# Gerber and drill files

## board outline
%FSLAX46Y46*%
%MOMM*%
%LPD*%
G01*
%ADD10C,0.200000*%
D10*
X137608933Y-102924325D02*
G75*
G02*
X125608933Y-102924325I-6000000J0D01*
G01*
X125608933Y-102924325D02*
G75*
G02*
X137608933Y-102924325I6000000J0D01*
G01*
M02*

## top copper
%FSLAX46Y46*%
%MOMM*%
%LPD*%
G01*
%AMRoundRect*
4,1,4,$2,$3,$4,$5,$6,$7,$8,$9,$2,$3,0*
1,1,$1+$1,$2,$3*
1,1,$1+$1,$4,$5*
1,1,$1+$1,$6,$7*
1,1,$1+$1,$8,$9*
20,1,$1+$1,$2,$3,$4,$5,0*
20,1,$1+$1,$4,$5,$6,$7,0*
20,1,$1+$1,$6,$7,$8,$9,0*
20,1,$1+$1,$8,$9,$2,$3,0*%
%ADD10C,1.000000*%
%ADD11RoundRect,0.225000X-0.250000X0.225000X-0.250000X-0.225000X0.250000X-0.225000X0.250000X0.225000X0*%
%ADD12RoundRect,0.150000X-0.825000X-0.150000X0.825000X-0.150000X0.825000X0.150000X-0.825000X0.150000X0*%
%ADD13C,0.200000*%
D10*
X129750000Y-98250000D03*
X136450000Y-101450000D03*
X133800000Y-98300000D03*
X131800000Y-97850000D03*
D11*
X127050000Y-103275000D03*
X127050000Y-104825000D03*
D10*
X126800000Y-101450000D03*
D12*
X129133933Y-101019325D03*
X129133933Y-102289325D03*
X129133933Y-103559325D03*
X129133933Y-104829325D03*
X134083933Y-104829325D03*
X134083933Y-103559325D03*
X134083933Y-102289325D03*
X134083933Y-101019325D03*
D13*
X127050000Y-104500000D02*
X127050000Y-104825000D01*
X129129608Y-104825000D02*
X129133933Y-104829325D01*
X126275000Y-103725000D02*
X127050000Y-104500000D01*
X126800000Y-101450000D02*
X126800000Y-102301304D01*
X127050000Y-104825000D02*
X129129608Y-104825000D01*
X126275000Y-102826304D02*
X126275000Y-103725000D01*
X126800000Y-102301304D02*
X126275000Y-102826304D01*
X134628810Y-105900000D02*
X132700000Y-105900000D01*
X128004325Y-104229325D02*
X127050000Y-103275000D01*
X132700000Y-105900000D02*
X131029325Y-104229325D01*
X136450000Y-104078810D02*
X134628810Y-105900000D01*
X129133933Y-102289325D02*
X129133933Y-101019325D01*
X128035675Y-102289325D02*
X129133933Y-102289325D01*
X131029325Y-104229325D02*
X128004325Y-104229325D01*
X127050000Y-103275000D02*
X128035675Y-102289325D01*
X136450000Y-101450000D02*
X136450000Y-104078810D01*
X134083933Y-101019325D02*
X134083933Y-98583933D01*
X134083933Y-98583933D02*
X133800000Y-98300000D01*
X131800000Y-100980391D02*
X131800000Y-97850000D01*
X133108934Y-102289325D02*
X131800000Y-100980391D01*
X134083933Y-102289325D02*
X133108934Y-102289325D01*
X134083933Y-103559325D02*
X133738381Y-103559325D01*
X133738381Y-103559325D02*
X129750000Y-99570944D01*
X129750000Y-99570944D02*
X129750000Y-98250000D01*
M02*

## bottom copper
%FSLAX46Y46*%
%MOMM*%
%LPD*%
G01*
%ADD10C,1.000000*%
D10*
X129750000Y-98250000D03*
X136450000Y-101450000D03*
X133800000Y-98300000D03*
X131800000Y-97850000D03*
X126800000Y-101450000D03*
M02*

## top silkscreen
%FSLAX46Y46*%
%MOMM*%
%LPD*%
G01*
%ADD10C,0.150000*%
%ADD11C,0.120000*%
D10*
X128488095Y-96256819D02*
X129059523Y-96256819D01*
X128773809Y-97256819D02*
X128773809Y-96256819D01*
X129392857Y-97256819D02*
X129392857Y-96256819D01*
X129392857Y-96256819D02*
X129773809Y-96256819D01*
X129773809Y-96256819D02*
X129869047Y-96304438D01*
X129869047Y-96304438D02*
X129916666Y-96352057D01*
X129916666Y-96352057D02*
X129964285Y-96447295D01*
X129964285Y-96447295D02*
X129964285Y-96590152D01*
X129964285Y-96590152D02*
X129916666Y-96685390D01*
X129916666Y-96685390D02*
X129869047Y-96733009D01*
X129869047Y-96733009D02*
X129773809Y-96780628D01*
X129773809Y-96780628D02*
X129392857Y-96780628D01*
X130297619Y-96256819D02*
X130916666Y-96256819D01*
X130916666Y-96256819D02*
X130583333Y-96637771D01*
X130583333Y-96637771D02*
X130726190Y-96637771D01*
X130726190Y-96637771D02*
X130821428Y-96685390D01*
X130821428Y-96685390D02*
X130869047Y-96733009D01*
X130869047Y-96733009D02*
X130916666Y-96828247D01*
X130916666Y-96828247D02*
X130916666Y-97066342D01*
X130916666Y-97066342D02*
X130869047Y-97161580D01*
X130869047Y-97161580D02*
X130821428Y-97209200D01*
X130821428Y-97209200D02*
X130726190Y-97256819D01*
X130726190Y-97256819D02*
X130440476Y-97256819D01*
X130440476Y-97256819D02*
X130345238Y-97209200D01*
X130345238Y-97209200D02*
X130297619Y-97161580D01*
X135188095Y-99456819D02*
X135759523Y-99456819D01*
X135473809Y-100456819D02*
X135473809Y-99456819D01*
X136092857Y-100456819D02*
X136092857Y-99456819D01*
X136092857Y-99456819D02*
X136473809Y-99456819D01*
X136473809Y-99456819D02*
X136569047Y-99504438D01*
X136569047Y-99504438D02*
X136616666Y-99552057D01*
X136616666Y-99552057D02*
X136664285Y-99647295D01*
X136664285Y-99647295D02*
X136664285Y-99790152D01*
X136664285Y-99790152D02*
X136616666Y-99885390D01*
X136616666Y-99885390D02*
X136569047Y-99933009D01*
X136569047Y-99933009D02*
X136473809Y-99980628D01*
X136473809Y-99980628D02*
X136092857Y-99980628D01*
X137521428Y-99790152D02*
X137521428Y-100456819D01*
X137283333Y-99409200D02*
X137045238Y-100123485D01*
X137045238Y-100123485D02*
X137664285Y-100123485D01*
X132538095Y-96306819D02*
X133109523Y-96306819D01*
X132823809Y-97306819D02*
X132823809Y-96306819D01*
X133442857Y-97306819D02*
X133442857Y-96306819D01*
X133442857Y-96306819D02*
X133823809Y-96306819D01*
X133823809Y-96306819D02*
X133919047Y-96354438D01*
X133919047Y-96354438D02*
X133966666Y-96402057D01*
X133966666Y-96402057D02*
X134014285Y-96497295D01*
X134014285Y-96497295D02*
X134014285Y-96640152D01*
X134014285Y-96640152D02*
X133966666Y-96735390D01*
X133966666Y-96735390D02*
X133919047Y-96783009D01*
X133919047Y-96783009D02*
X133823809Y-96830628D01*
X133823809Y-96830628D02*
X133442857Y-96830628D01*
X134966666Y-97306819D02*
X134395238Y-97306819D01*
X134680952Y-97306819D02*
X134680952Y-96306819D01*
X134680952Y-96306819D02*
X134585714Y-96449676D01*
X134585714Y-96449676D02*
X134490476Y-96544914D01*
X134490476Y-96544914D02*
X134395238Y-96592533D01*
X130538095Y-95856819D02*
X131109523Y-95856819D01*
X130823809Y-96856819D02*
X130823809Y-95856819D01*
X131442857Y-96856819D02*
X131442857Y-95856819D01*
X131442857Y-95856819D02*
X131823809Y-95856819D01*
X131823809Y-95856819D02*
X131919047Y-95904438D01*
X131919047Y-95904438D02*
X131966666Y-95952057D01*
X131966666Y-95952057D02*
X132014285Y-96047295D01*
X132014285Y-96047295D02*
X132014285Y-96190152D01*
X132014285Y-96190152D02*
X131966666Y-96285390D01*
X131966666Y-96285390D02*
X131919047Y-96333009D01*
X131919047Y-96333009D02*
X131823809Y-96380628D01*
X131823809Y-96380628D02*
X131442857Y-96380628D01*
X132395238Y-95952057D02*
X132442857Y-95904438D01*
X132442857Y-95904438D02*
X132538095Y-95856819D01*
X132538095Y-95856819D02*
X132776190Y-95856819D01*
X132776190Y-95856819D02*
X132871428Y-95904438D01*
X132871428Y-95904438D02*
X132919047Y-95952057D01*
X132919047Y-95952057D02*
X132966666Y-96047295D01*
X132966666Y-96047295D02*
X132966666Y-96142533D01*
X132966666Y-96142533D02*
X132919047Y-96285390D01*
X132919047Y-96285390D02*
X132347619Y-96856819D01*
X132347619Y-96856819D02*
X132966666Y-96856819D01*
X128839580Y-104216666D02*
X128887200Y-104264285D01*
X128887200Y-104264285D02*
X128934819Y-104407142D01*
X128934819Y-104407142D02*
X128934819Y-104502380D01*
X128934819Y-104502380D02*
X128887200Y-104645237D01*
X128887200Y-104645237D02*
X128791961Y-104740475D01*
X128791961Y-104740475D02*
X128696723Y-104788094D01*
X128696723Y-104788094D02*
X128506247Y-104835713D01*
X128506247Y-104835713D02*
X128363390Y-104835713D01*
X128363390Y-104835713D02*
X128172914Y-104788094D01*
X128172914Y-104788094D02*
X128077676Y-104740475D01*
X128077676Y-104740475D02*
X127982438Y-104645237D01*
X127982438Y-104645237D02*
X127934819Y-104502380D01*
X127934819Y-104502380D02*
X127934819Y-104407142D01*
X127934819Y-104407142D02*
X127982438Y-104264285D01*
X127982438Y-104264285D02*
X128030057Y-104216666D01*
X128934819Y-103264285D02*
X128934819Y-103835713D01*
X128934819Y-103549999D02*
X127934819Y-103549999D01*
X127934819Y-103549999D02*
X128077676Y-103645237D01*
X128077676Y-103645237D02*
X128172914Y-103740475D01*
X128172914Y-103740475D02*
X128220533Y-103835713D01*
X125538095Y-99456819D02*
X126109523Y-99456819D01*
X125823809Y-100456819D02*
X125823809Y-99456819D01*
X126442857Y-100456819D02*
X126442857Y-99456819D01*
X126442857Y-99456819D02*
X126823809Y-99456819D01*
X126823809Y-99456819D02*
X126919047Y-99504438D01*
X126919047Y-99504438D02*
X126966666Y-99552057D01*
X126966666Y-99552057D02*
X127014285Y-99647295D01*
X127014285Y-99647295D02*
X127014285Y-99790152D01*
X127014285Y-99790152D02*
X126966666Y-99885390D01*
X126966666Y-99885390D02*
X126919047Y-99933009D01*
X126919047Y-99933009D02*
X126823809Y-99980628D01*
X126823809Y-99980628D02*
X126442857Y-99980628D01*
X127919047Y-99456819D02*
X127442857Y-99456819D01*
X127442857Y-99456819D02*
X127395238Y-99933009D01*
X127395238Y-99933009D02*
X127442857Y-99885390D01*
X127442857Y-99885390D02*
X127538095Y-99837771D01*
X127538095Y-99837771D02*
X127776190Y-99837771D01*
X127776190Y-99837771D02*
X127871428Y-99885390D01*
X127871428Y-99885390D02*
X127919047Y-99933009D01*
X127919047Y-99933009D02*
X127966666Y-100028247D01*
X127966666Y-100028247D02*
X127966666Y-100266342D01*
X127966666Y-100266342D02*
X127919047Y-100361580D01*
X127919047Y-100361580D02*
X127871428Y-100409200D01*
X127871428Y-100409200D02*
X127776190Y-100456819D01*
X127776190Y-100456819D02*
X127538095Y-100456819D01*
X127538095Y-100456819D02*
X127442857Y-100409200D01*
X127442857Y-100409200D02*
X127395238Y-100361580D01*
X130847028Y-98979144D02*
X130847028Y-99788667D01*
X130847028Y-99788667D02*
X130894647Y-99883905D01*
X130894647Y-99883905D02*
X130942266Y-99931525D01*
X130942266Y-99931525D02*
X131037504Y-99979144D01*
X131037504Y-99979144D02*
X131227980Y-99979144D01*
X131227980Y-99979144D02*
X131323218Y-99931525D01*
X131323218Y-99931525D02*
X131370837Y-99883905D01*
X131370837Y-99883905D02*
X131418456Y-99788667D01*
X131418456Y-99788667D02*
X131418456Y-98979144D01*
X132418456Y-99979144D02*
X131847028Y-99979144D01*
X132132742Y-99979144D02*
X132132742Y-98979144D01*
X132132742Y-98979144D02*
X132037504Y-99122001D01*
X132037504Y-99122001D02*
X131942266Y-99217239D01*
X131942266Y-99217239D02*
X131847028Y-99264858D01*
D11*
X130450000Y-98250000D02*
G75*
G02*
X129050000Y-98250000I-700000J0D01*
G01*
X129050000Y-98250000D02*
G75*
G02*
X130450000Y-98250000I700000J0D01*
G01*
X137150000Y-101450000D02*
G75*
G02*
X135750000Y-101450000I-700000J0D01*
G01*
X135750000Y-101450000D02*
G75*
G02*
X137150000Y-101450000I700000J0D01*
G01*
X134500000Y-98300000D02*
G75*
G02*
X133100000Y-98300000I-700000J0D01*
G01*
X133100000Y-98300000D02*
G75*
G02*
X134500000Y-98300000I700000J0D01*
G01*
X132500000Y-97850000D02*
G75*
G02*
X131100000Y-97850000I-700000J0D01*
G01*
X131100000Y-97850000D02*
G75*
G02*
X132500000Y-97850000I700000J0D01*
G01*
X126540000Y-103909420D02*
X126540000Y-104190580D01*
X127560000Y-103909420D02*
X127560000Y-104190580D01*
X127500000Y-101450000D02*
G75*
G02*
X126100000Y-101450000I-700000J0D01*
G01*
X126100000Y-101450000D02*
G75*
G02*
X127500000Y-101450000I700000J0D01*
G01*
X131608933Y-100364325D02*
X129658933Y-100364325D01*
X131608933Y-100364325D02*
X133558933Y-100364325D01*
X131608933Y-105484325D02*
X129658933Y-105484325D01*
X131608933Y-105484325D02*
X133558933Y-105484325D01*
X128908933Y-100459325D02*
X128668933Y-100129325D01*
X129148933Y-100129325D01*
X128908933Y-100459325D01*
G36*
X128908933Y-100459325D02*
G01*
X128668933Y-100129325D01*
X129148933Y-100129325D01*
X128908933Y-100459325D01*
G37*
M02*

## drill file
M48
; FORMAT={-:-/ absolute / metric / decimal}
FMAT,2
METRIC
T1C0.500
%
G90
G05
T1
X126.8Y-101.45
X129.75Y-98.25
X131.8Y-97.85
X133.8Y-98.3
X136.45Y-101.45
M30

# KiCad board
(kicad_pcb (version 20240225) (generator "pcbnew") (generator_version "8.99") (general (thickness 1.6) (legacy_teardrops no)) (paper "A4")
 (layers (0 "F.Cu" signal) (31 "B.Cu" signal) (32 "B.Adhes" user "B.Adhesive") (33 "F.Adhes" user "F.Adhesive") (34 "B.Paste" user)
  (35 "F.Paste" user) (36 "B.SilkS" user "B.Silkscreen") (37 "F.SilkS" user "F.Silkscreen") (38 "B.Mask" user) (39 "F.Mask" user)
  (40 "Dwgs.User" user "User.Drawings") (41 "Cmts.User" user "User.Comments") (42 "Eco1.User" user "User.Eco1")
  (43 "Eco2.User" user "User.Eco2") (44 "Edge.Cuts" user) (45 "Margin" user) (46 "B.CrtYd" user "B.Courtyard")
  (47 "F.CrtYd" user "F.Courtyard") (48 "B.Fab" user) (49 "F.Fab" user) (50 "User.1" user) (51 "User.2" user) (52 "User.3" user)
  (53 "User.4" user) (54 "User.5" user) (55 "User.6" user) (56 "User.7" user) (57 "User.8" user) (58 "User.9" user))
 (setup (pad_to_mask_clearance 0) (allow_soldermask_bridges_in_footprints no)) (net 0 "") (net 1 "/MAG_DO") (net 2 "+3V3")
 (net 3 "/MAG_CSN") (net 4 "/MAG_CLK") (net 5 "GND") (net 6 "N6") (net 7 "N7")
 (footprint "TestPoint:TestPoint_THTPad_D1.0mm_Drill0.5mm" (layer "F.Cu") (at 129.75 98.25)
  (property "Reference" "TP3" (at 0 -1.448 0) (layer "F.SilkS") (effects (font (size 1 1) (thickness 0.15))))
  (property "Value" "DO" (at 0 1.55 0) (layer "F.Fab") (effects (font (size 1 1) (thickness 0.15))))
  (fp_circle (center 0 0) (end 0 0.7) (stroke (width 0.12) (type solid)) (fill none) (layer "F.SilkS"))
  (pad "1" thru_hole circle (at 0 0) (size 1 1) (drill 0.5) (layers "*.Cu" "*.Mask") (remove_unused_layers no) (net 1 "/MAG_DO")))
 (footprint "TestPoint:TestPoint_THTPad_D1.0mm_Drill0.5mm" (layer "F.Cu") (at 136.45 101.45)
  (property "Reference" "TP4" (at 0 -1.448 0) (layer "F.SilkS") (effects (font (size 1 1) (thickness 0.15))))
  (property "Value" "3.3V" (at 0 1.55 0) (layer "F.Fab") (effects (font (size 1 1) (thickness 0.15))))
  (fp_circle (center 0 0) (end 0 0.7) (stroke (width 0.12) (type solid)) (fill none) (layer "F.SilkS"))
  (pad "1" thru_hole circle (at 0 0) (size 1 1) (drill 0.5) (layers "*.Cu" "*.Mask") (remove_unused_layers no) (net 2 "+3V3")))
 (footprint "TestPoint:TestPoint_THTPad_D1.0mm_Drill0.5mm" (layer "F.Cu") (at 133.8 98.3)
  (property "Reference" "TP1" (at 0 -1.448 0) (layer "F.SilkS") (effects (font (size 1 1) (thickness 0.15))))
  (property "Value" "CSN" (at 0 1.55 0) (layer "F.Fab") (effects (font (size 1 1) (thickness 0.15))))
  (fp_circle (center 0 0) (end 0 0.7) (stroke (width 0.12) (type solid)) (fill none) (layer "F.SilkS"))
  (pad "1" thru_hole circle (at 0 0) (size 1 1) (drill 0.5) (layers "*.Cu" "*.Mask") (remove_unused_layers no) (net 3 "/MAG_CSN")))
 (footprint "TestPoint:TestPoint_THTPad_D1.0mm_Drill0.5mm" (layer "F.Cu") (at 131.8 97.85)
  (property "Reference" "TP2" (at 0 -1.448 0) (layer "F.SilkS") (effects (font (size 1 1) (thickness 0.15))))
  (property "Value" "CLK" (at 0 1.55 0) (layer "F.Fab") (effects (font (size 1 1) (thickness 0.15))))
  (fp_circle (center 0 0) (end 0 0.7) (stroke (width 0.12) (type solid)) (fill none) (layer "F.SilkS"))
  (pad "1" thru_hole circle (at 0 0) (size 1 1) (drill 0.5) (layers "*.Cu" "*.Mask") (remove_unused_layers no) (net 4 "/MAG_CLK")))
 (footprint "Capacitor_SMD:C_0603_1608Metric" (layer "F.Cu") (at 127.05 104.05 -90)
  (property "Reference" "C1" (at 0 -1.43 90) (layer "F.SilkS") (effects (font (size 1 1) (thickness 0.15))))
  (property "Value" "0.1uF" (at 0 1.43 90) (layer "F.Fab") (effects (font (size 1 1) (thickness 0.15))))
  (fp_line (start -0.14058 0.51) (end 0.14058 0.51) (stroke (width 0.12) (type solid)) (layer "F.SilkS"))
  (fp_line (start -0.14058 -0.51) (end 0.14058 -0.51) (stroke (width 0.12) (type solid)) (layer "F.SilkS"))
  (pad "1" smd roundrect (at -0.775 0 270) (size 0.9 0.95) (layers "F.Cu" "F.Paste" "F.Mask") (roundrect_rratio 0.25) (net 2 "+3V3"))
  (pad "2" smd roundrect (at 0.775 0 270) (size 0.9 0.95) (layers "F.Cu" "F.Paste" "F.Mask") (roundrect_rratio 0.25) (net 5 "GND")))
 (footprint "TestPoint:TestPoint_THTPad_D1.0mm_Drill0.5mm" (layer "F.Cu") (at 126.8 101.45)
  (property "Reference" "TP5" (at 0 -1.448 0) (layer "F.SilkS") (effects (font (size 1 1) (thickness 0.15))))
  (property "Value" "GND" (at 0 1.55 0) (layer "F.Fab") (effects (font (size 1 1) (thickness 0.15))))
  (fp_circle (center 0 0) (end 0 0.7) (stroke (width 0.12) (type solid)) (fill none) (layer "F.SilkS"))
  (pad "1" thru_hole circle (at 0 0) (size 1 1) (drill 0.5) (layers "*.Cu" "*.Mask") (remove_unused_layers no) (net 5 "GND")))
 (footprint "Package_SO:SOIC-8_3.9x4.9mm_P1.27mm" (layer "F.Cu") (at 131.608933 102.924325)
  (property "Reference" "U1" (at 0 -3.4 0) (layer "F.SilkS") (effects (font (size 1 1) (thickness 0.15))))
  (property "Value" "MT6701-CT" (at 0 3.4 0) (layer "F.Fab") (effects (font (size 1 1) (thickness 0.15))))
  (fp_line (start 0 -2.56) (end -1.95 -2.56) (stroke (width 0.12) (type solid)) (layer "F.SilkS"))
  (fp_line (start 0 -2.56) (end 1.95 -2.56) (stroke (width 0.12) (type solid)) (layer "F.SilkS"))
  (fp_line (start 0 2.56) (end -1.95 2.56) (stroke (width 0.12) (type solid)) (layer "F.SilkS"))
  (fp_line (start 0 2.56) (end 1.95 2.56) (stroke (width 0.12) (type solid)) (layer "F.SilkS"))
  (fp_poly
   (pts (xy -2.7 -2.465) (xy -2.94 -2.795) (xy -2.46 -2.795) (xy -2.7 -2.465)) (stroke (width 0.12) (type solid)) (fill solid)
   (layer "F.SilkS"))
  (pad "1" smd roundrect (at -2.475 -1.905) (size 1.95 0.6) (layers "F.Cu" "F.Paste" "F.Mask") (roundrect_rratio 0.25) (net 2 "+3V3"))
  (pad "2" smd roundrect (at -2.475 -0.635) (size 1.95 0.6) (layers "F.Cu" "F.Paste" "F.Mask") (roundrect_rratio 0.25) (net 2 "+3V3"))
  (pad "3" smd roundrect (at -2.475 0.635) (size 1.95 0.6) (layers "F.Cu" "F.Paste" "F.Mask") (roundrect_rratio 0.25) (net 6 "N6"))
  (pad "4" smd roundrect (at -2.475 1.905) (size 1.95 0.6) (layers "F.Cu" "F.Paste" "F.Mask") (roundrect_rratio 0.25) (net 5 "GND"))
  (pad "5" smd roundrect (at 2.475 1.905) (size 1.95 0.6) (layers "F.Cu" "F.Paste" "F.Mask") (roundrect_rratio 0.25) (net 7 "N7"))
  (pad "6" smd roundrect (at 2.475 0.635) (size 1.95 0.6) (layers "F.Cu" "F.Paste" "F.Mask") (roundrect_rratio 0.25) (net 1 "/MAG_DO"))
  (pad "7" smd roundrect (at 2.475 -0.635) (size 1.95 0.6) (layers "F.Cu" "F.Paste" "F.Mask") (roundrect_rratio 0.25) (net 4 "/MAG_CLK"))
  (pad "8" smd roundrect (at 2.475 -1.905) (size 1.95 0.6) (layers "F.Cu" "F.Paste" "F.Mask") (roundrect_rratio 0.25) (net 3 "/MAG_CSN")))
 (gr_circle (center 131.608933 102.924325) (end 137.608933 102.924325) (stroke (width 0.2) (type default)) (fill none) (layer "Edge.Cuts"))
 (segment (start 127.05 104.5) (end 127.05 104.825) (width 0.2) (layer "F.Cu") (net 5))
 (segment (start 129.129608 104.825) (end 129.133933 104.829325) (width 0.2) (layer "F.Cu") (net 5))
 (segment (start 126.275 103.725) (end 127.05 104.5) (width 0.2) (layer "F.Cu") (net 5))
 (segment (start 126.8 101.45) (end 126.8 102.301304) (width 0.2) (layer "F.Cu") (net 5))
 (segment (start 127.05 104.825) (end 129.129608 104.825) (width 0.2) (layer "F.Cu") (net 5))
 (segment (start 126.275 102.826304) (end 126.275 103.725) (width 0.2) (layer "F.Cu") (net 5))
 (segment (start 126.8 102.301304) (end 126.275 102.826304) (width 0.2) (layer "F.Cu") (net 5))
 (segment (start 134.62881 105.9) (end 132.7 105.9) (width 0.2) (layer "F.Cu") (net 2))
 (segment (start 128.004325 104.229325) (end 127.05 103.275) (width 0.2) (layer "F.Cu") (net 2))
 (segment (start 132.7 105.9) (end 131.029325 104.229325) (width 0.2) (layer "F.Cu") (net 2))
 (segment (start 136.45 104.07881) (end 134.62881 105.9) (width 0.2) (layer "F.Cu") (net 2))
 (segment (start 129.133933 102.289325) (end 129.133933 101.019325) (width 0.2) (layer "F.Cu") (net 2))
 (segment (start 128.035675 102.289325) (end 129.133933 102.289325) (width 0.2) (layer "F.Cu") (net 2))
 (segment (start 131.029325 104.229325) (end 128.004325 104.229325) (width 0.2) (layer "F.Cu") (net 2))
 (segment (start 127.05 103.275) (end 128.035675 102.289325) (width 0.2) (layer "F.Cu") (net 2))
 (segment (start 136.45 101.45) (end 136.45 104.07881) (width 0.2) (layer "F.Cu") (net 2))
 (segment (start 134.083933 101.019325) (end 134.083933 98.583933) (width 0.2) (layer "F.Cu") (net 3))
 (segment (start 134.083933 98.583933) (end 133.8 98.3) (width 0.2) (layer "F.Cu") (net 3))
 (segment (start 131.8 100.980391) (end 131.8 97.85) (width 0.2) (layer "F.Cu") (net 4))
 (segment (start 133.108934 102.289325) (end 131.8 100.980391) (width 0.2) (layer "F.Cu") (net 4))
 (segment (start 134.083933 102.289325) (end 133.108934 102.289325) (width 0.2) (layer "F.Cu") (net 4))
 (segment (start 134.083933 103.559325) (end 133.738381 103.559325) (width 0.2) (layer "F.Cu") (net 1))
 (segment (start 133.738381 103.559325) (end 129.75 99.570944) (width 0.2) (layer "F.Cu") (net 1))
 (segment (start 129.75 99.570944) (end 129.75 98.25) (width 0.2) (layer "F.Cu") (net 1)))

